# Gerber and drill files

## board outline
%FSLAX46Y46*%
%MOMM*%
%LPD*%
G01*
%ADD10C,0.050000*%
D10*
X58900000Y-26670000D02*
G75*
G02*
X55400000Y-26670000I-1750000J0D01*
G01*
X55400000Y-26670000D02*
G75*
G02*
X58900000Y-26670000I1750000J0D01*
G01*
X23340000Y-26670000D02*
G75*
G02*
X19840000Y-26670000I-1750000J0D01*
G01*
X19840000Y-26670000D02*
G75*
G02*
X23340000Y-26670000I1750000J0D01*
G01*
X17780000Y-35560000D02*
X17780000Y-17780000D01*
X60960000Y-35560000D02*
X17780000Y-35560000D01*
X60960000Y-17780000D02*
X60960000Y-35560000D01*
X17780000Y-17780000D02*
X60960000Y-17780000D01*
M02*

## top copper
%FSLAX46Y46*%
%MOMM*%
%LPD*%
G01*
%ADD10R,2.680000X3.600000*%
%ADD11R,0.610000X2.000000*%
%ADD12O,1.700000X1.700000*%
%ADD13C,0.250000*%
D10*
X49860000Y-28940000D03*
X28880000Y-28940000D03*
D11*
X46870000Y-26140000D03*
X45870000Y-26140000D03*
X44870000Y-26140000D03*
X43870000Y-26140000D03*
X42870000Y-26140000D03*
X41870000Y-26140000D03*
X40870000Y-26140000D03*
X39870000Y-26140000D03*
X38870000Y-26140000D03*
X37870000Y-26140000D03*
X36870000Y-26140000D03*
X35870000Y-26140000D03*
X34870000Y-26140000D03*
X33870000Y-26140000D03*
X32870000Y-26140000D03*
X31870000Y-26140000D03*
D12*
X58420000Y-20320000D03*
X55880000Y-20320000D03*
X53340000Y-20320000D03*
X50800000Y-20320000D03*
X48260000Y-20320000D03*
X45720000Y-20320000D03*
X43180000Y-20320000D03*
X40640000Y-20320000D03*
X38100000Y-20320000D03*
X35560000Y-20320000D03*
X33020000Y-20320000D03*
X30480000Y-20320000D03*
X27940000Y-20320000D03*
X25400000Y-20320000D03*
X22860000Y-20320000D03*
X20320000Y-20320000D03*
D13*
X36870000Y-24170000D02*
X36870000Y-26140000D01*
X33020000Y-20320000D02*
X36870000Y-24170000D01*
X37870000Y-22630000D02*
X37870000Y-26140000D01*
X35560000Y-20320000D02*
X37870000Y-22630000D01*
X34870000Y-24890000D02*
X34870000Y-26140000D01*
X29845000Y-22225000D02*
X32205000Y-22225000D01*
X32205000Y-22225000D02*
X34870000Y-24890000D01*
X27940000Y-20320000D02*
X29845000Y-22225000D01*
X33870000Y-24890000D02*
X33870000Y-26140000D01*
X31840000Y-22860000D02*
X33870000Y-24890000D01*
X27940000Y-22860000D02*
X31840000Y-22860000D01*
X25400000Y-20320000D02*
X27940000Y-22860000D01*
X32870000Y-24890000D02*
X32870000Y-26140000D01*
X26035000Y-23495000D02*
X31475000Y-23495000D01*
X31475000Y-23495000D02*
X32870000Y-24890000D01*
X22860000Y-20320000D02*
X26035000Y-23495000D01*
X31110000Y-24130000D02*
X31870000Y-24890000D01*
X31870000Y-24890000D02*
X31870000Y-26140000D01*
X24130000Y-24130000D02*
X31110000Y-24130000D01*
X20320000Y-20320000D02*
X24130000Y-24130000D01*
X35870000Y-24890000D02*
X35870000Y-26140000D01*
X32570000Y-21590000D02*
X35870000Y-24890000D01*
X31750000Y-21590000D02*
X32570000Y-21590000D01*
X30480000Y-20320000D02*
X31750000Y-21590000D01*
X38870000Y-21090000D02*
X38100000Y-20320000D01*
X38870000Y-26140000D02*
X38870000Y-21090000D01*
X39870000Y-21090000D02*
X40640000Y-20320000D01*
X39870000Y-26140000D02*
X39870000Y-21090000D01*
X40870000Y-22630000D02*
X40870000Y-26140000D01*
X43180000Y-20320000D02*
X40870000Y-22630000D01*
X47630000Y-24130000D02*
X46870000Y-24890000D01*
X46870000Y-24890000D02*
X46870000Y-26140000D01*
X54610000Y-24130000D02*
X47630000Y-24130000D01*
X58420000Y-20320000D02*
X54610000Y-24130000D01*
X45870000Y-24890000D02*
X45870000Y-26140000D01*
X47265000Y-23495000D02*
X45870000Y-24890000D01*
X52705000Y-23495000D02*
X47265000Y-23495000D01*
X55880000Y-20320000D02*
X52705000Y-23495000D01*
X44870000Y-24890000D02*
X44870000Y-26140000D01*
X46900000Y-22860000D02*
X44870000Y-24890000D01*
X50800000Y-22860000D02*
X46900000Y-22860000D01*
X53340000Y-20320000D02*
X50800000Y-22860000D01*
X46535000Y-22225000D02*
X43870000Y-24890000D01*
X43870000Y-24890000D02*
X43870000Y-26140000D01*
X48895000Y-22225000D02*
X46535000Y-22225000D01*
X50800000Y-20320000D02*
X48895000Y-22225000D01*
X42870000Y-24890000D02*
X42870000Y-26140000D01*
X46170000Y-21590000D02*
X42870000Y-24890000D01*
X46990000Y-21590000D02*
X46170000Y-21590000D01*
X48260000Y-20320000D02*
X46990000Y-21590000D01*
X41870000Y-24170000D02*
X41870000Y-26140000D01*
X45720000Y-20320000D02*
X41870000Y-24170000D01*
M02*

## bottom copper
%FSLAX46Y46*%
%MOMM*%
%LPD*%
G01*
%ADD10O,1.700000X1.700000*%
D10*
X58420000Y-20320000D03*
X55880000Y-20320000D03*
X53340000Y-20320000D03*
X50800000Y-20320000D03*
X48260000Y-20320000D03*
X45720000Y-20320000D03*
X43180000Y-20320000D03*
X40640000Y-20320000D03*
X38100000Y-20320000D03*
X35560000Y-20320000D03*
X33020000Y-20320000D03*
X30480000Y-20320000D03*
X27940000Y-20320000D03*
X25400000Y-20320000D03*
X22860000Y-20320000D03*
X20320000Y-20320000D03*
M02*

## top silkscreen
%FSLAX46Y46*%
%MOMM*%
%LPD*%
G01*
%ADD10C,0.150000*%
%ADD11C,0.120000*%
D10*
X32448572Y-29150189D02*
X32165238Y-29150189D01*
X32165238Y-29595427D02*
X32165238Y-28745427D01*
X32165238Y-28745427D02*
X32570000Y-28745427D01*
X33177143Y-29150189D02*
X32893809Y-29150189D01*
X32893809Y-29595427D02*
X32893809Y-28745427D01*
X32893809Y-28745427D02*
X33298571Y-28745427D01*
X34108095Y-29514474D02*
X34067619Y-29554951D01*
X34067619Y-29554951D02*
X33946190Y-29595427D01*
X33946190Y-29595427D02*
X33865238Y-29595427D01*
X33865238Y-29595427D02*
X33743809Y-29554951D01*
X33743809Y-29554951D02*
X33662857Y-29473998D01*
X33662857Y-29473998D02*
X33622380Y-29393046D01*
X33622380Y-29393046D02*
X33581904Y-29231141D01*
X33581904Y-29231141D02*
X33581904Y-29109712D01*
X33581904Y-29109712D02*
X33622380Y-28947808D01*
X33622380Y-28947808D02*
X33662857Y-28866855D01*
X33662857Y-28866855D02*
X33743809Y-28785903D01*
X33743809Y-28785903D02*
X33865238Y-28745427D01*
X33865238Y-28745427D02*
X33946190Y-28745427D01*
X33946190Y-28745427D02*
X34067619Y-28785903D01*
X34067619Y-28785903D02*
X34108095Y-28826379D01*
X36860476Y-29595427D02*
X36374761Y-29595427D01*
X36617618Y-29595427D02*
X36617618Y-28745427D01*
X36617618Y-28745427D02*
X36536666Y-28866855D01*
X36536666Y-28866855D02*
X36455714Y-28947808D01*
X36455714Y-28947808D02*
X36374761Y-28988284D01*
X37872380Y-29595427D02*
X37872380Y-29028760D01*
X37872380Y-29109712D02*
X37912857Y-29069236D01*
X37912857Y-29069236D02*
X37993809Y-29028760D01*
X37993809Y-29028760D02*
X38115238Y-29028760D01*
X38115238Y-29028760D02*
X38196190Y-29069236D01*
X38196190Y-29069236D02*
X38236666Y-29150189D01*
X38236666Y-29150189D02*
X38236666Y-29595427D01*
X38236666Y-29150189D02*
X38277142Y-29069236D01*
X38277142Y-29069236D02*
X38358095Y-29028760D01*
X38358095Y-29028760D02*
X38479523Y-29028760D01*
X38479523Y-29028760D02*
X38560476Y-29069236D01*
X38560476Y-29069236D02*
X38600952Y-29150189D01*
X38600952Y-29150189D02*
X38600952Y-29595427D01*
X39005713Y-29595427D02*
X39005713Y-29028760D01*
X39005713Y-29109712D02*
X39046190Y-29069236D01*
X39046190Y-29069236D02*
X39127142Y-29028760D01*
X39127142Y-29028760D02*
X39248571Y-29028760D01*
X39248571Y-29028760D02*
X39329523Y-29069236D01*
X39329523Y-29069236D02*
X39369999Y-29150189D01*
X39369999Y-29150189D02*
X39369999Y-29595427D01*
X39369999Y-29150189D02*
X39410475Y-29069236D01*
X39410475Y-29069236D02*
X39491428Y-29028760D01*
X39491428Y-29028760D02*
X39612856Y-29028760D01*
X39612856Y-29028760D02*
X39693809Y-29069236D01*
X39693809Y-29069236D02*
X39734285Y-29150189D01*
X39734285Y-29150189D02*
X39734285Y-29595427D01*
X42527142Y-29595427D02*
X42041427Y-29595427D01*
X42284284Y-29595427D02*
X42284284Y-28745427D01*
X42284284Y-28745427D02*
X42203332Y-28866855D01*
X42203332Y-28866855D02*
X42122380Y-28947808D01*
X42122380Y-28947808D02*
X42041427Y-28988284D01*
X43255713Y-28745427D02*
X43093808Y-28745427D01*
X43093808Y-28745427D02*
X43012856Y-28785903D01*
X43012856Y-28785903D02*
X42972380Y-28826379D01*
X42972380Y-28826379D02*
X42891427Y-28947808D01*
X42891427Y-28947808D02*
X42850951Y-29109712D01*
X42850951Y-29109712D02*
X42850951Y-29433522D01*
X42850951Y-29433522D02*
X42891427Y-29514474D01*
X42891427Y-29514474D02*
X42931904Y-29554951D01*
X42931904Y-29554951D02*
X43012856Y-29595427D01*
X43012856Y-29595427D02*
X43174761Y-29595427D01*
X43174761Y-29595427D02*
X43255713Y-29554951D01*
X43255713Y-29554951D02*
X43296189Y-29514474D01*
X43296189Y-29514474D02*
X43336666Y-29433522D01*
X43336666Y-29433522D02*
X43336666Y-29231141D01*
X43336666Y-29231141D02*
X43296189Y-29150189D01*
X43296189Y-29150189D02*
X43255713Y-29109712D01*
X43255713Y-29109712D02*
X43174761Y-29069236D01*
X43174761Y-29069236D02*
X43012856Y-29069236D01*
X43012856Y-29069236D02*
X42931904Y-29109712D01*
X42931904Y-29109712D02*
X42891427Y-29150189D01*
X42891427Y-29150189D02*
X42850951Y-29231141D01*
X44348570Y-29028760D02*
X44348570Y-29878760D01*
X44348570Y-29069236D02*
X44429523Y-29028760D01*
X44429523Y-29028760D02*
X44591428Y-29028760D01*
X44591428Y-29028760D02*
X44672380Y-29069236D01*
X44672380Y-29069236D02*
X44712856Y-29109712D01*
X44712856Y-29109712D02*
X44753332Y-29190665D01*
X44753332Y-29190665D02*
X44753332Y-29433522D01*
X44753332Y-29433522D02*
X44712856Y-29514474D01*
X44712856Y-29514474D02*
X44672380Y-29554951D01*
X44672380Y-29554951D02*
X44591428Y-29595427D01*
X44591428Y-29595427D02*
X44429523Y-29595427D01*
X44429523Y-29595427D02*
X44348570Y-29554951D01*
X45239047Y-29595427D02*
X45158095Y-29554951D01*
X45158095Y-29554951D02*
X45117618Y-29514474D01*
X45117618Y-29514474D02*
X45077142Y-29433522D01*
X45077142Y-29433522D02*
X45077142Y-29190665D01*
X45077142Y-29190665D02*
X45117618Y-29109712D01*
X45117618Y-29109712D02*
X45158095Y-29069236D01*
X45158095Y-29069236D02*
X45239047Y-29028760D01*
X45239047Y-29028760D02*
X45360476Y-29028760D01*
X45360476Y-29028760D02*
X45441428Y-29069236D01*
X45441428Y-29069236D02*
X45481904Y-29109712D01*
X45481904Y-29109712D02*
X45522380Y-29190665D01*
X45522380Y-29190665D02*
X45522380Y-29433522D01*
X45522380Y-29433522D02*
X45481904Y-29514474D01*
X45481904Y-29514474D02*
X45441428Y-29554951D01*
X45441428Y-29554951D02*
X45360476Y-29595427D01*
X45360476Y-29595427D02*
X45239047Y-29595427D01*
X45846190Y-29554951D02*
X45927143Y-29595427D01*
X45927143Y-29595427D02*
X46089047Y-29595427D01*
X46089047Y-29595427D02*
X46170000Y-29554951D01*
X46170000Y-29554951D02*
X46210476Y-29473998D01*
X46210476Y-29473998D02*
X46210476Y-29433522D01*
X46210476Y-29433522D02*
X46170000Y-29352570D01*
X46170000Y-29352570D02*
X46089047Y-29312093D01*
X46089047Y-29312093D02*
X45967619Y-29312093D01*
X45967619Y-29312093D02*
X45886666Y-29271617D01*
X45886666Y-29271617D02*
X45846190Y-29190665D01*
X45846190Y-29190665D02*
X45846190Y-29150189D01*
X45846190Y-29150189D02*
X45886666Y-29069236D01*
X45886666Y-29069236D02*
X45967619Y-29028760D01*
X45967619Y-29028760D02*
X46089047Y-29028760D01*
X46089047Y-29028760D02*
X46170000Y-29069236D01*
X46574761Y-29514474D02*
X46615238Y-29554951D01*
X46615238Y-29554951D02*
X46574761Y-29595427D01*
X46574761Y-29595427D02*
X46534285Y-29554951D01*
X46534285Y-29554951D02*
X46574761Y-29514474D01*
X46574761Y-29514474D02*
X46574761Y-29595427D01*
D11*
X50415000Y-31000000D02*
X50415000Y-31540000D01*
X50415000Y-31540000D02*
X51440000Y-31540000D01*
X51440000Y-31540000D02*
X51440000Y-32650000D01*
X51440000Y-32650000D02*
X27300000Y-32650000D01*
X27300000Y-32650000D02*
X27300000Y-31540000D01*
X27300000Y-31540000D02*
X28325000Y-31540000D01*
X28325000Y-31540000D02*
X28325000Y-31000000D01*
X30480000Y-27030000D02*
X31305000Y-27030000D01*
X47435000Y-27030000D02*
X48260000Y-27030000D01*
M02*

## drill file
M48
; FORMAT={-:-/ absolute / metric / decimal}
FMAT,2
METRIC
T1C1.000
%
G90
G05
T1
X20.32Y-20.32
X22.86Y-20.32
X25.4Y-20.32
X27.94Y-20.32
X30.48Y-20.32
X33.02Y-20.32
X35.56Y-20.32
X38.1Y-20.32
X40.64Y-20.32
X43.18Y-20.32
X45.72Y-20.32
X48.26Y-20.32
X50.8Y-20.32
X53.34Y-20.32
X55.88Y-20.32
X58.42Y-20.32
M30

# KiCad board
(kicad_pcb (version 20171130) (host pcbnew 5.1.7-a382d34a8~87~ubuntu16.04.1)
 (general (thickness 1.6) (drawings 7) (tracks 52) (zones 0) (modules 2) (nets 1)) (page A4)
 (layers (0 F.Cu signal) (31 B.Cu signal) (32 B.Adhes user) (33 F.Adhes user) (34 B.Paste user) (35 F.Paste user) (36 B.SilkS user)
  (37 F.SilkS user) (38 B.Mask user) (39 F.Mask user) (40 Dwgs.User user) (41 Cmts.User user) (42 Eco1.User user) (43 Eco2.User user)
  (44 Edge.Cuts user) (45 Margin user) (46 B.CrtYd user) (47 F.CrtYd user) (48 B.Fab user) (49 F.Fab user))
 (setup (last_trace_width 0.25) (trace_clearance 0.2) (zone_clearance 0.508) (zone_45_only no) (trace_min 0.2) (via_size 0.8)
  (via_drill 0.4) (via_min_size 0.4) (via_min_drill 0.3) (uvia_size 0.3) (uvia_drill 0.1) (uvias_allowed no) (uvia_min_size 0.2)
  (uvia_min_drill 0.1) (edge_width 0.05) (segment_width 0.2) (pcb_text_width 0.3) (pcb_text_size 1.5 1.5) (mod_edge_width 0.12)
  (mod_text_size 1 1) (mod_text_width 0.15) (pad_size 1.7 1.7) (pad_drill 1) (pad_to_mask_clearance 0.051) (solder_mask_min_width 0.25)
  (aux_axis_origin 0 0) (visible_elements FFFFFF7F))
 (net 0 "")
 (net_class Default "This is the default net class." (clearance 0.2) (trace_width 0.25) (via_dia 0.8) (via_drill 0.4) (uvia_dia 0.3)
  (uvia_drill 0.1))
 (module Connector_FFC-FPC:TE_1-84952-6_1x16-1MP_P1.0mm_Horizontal (layer F.Cu) (at 39.37 27.94)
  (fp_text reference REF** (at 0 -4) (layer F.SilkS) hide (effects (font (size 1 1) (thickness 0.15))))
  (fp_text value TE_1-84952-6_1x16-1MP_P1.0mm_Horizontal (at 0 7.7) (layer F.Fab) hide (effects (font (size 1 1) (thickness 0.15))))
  (fp_line (start 11.045 3.06) (end 11.045 3.6) (layer F.SilkS) (width 0.12))
  (fp_line (start 11.045 3.6) (end 12.07 3.6) (layer F.SilkS) (width 0.12))
  (fp_line (start 12.07 3.6) (end 12.07 4.71) (layer F.SilkS) (width 0.12))
  (fp_line (start 12.07 4.71) (end -12.07 4.71) (layer F.SilkS) (width 0.12))
  (fp_line (start -12.07 4.71) (end -12.07 3.6) (layer F.SilkS) (width 0.12))
  (fp_line (start -12.07 3.6) (end -11.045 3.6) (layer F.SilkS) (width 0.12))
  (fp_line (start -11.045 3.6) (end -11.045 3.06) (layer F.SilkS) (width 0.12))
  (fp_line (start -8.89 -0.91) (end -8.065 -0.91) (layer F.SilkS) (width 0.12))
  (fp_line (start 8.065 -0.91) (end 8.89 -0.91) (layer F.SilkS) (width 0.12))
  (pad MP smd rect (at 10.49 1) (size 2.68 3.6) (layers F.Cu F.Paste F.Mask))
  (pad MP smd rect (at -10.49 1) (size 2.68 3.6) (layers F.Cu F.Paste F.Mask))
  (pad 16 smd rect (at 7.5 -1.8) (size 0.61 2) (layers F.Cu F.Paste F.Mask))
  (pad 15 smd rect (at 6.5 -1.8) (size 0.61 2) (layers F.Cu F.Paste F.Mask))
  (pad 14 smd rect (at 5.5 -1.8) (size 0.61 2) (layers F.Cu F.Paste F.Mask))
  (pad 13 smd rect (at 4.5 -1.8) (size 0.61 2) (layers F.Cu F.Paste F.Mask))
  (pad 12 smd rect (at 3.5 -1.8) (size 0.61 2) (layers F.Cu F.Paste F.Mask))
  (pad 11 smd rect (at 2.5 -1.8) (size 0.61 2) (layers F.Cu F.Paste F.Mask))
  (pad 10 smd rect (at 1.5 -1.8) (size 0.61 2) (layers F.Cu F.Paste F.Mask))
  (pad 9 smd rect (at 0.5 -1.8) (size 0.61 2) (layers F.Cu F.Paste F.Mask))
  (pad 8 smd rect (at -0.5 -1.8) (size 0.61 2) (layers F.Cu F.Paste F.Mask))
  (pad 7 smd rect (at -1.5 -1.8) (size 0.61 2) (layers F.Cu F.Paste F.Mask))
  (pad 6 smd rect (at -2.5 -1.8) (size 0.61 2) (layers F.Cu F.Paste F.Mask))
  (pad 5 smd rect (at -3.5 -1.8) (size 0.61 2) (layers F.Cu F.Paste F.Mask))
  (pad 4 smd rect (at -4.5 -1.8) (size 0.61 2) (layers F.Cu F.Paste F.Mask))
  (pad 3 smd rect (at -5.5 -1.8) (size 0.61 2) (layers F.Cu F.Paste F.Mask))
  (pad 2 smd rect (at -6.5 -1.8) (size 0.61 2) (layers F.Cu F.Paste F.Mask))
  (pad 1 smd rect (at -7.5 -1.8) (size 0.61 2) (layers F.Cu F.Paste F.Mask)))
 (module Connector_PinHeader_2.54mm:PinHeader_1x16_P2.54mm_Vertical (layer F.Cu) (at 20.32 20.32 90)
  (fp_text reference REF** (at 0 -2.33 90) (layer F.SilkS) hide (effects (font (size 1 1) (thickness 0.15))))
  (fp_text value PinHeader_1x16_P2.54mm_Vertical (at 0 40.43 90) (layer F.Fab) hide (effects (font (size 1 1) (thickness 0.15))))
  (pad 16 thru_hole oval (at 0 38.1 90) (size 1.7 1.7) (drill 1) (layers *.Cu *.Mask))
  (pad 15 thru_hole oval (at 0 35.56 90) (size 1.7 1.7) (drill 1) (layers *.Cu *.Mask))
  (pad 14 thru_hole oval (at 0 33.02 90) (size 1.7 1.7) (drill 1) (layers *.Cu *.Mask))
  (pad 13 thru_hole oval (at 0 30.48 90) (size 1.7 1.7) (drill 1) (layers *.Cu *.Mask))
  (pad 12 thru_hole oval (at 0 27.94 90) (size 1.7 1.7) (drill 1) (layers *.Cu *.Mask))
  (pad 11 thru_hole oval (at 0 25.4 90) (size 1.7 1.7) (drill 1) (layers *.Cu *.Mask))
  (pad 10 thru_hole oval (at 0 22.86 90) (size 1.7 1.7) (drill 1) (layers *.Cu *.Mask))
  (pad 9 thru_hole oval (at 0 20.32 90) (size 1.7 1.7) (drill 1) (layers *.Cu *.Mask))
  (pad 8 thru_hole oval (at 0 17.78 90) (size 1.7 1.7) (drill 1) (layers *.Cu *.Mask))
  (pad 7 thru_hole oval (at 0 15.24 90) (size 1.7 1.7) (drill 1) (layers *.Cu *.Mask))
  (pad 6 thru_hole oval (at 0 12.7 90) (size 1.7 1.7) (drill 1) (layers *.Cu *.Mask))
  (pad 5 thru_hole oval (at 0 10.16 90) (size 1.7 1.7) (drill 1) (layers *.Cu *.Mask))
  (pad 4 thru_hole oval (at 0 7.62 90) (size 1.7 1.7) (drill 1) (layers *.Cu *.Mask))
  (pad 3 thru_hole oval (at 0 5.08 90) (size 1.7 1.7) (drill 1) (layers *.Cu *.Mask))
  (pad 2 thru_hole oval (at 0 2.54 90) (size 1.7 1.7) (drill 1) (layers *.Cu *.Mask))
  (pad 1 thru_hole oval (at 0 0 90) (size 1.7 1.7) (drill 1) (layers *.Cu *.Mask)))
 (gr_circle (center 57.15 26.67) (end 58.9 26.67) (layer Edge.Cuts) (width 0.05))
 (gr_circle (center 21.59 26.67) (end 23.34 26.67) (layer Edge.Cuts) (width 0.05))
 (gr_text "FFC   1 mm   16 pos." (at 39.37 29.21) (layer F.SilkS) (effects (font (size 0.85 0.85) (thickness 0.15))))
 (gr_line (start 17.78 35.56) (end 17.78 17.78) (layer Edge.Cuts) (width 0.05))
 (gr_line (start 60.96 35.56) (end 17.78 35.56) (layer Edge.Cuts) (width 0.05))
 (gr_line (start 60.96 17.78) (end 60.96 35.56) (layer Edge.Cuts) (width 0.05))
 (gr_line (start 17.78 17.78) (end 60.96 17.78) (layer Edge.Cuts) (width 0.05))
 (segment (start 36.87 24.17) (end 36.87 26.14) (width 0.25) (layer F.Cu) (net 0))
 (segment (start 33.02 20.32) (end 36.87 24.17) (width 0.25) (layer F.Cu) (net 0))
 (segment (start 37.87 22.63) (end 37.87 26.14) (width 0.25) (layer F.Cu) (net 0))
 (segment (start 35.56 20.32) (end 37.87 22.63) (width 0.25) (layer F.Cu) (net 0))
 (segment (start 34.87 24.89) (end 34.87 26.14) (width 0.25) (layer F.Cu) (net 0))
 (segment (start 29.845 22.225) (end 32.205 22.225) (width 0.25) (layer F.Cu) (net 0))
 (segment (start 32.205 22.225) (end 34.87 24.89) (width 0.25) (layer F.Cu) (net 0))
 (segment (start 27.94 20.32) (end 29.845 22.225) (width 0.25) (layer F.Cu) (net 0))
 (segment (start 33.87 24.89) (end 33.87 26.14) (width 0.25) (layer F.Cu) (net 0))
 (segment (start 31.84 22.86) (end 33.87 24.89) (width 0.25) (layer F.Cu) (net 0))
 (segment (start 27.94 22.86) (end 31.84 22.86) (width 0.25) (layer F.Cu) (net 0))
 (segment (start 25.4 20.32) (end 27.94 22.86) (width 0.25) (layer F.Cu) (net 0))
 (segment (start 32.87 24.89) (end 32.87 26.14) (width 0.25) (layer F.Cu) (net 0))
 (segment (start 26.035 23.495) (end 31.475 23.495) (width 0.25) (layer F.Cu) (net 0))
 (segment (start 31.475 23.495) (end 32.87 24.89) (width 0.25) (layer F.Cu) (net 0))
 (segment (start 22.86 20.32) (end 26.035 23.495) (width 0.25) (layer F.Cu) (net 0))
 (segment (start 31.11 24.13) (end 31.87 24.89) (width 0.25) (layer F.Cu) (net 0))
 (segment (start 31.87 24.89) (end 31.87 26.14) (width 0.25) (layer F.Cu) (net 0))
 (segment (start 24.13 24.13) (end 31.11 24.13) (width 0.25) (layer F.Cu) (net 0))
 (segment (start 20.32 20.32) (end 24.13 24.13) (width 0.25) (layer F.Cu) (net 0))
 (segment (start 35.87 24.89) (end 35.87 26.14) (width 0.25) (layer F.Cu) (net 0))
 (segment (start 32.57 21.59) (end 35.87 24.89) (width 0.25) (layer F.Cu) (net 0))
 (segment (start 31.75 21.59) (end 32.57 21.59) (width 0.25) (layer F.Cu) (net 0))
 (segment (start 30.48 20.32) (end 31.75 21.59) (width 0.25) (layer F.Cu) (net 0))
 (segment (start 38.87 21.09) (end 38.1 20.32) (width 0.25) (layer F.Cu) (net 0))
 (segment (start 38.87 26.14) (end 38.87 21.09) (width 0.25) (layer F.Cu) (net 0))
 (segment (start 39.87 21.09) (end 40.64 20.32) (width 0.25) (layer F.Cu) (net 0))
 (segment (start 39.87 26.14) (end 39.87 21.09) (width 0.25) (layer F.Cu) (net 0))
 (segment (start 40.87 22.63) (end 40.87 26.14) (width 0.25) (layer F.Cu) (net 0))
 (segment (start 43.18 20.32) (end 40.87 22.63) (width 0.25) (layer F.Cu) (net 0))
 (segment (start 47.63 24.13) (end 46.87 24.89) (width 0.25) (layer F.Cu) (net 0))
 (segment (start 46.87 24.89) (end 46.87 26.14) (width 0.25) (layer F.Cu) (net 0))
 (segment (start 54.61 24.13) (end 47.63 24.13) (width 0.25) (layer F.Cu) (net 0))
 (segment (start 58.42 20.32) (end 54.61 24.13) (width 0.25) (layer F.Cu) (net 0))
 (segment (start 45.87 24.89) (end 45.87 26.14) (width 0.25) (layer F.Cu) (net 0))
 (segment (start 47.265 23.495) (end 45.87 24.89) (width 0.25) (layer F.Cu) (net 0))
 (segment (start 52.705 23.495) (end 47.265 23.495) (width 0.25) (layer F.Cu) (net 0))
 (segment (start 55.88 20.32) (end 52.705 23.495) (width 0.25) (layer F.Cu) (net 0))
 (segment (start 44.87 24.89) (end 44.87 26.14) (width 0.25) (layer F.Cu) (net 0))
 (segment (start 46.9 22.86) (end 44.87 24.89) (width 0.25) (layer F.Cu) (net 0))
 (segment (start 50.8 22.86) (end 46.9 22.86) (width 0.25) (layer F.Cu) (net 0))
 (segment (start 53.34 20.32) (end 50.8 22.86) (width 0.25) (layer F.Cu) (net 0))
 (segment (start 46.535 22.225) (end 43.87 24.89) (width 0.25) (layer F.Cu) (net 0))
 (segment (start 43.87 24.89) (end 43.87 26.14) (width 0.25) (layer F.Cu) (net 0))
 (segment (start 48.895 22.225) (end 46.535 22.225) (width 0.25) (layer F.Cu) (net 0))
 (segment (start 50.8 20.32) (end 48.895 22.225) (width 0.25) (layer F.Cu) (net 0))
 (segment (start 42.87 24.89) (end 42.87 26.14) (width 0.25) (layer F.Cu) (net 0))
 (segment (start 46.17 21.59) (end 42.87 24.89) (width 0.25) (layer F.Cu) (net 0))
 (segment (start 46.99 21.59) (end 46.17 21.59) (width 0.25) (layer F.Cu) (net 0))
 (segment (start 48.26 20.32) (end 46.99 21.59) (width 0.25) (layer F.Cu) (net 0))
 (segment (start 41.87 24.17) (end 41.87 26.14) (width 0.25) (layer F.Cu) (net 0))
 (segment (start 45.72 20.32) (end 41.87 24.17) (width 0.25) (layer F.Cu) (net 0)))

